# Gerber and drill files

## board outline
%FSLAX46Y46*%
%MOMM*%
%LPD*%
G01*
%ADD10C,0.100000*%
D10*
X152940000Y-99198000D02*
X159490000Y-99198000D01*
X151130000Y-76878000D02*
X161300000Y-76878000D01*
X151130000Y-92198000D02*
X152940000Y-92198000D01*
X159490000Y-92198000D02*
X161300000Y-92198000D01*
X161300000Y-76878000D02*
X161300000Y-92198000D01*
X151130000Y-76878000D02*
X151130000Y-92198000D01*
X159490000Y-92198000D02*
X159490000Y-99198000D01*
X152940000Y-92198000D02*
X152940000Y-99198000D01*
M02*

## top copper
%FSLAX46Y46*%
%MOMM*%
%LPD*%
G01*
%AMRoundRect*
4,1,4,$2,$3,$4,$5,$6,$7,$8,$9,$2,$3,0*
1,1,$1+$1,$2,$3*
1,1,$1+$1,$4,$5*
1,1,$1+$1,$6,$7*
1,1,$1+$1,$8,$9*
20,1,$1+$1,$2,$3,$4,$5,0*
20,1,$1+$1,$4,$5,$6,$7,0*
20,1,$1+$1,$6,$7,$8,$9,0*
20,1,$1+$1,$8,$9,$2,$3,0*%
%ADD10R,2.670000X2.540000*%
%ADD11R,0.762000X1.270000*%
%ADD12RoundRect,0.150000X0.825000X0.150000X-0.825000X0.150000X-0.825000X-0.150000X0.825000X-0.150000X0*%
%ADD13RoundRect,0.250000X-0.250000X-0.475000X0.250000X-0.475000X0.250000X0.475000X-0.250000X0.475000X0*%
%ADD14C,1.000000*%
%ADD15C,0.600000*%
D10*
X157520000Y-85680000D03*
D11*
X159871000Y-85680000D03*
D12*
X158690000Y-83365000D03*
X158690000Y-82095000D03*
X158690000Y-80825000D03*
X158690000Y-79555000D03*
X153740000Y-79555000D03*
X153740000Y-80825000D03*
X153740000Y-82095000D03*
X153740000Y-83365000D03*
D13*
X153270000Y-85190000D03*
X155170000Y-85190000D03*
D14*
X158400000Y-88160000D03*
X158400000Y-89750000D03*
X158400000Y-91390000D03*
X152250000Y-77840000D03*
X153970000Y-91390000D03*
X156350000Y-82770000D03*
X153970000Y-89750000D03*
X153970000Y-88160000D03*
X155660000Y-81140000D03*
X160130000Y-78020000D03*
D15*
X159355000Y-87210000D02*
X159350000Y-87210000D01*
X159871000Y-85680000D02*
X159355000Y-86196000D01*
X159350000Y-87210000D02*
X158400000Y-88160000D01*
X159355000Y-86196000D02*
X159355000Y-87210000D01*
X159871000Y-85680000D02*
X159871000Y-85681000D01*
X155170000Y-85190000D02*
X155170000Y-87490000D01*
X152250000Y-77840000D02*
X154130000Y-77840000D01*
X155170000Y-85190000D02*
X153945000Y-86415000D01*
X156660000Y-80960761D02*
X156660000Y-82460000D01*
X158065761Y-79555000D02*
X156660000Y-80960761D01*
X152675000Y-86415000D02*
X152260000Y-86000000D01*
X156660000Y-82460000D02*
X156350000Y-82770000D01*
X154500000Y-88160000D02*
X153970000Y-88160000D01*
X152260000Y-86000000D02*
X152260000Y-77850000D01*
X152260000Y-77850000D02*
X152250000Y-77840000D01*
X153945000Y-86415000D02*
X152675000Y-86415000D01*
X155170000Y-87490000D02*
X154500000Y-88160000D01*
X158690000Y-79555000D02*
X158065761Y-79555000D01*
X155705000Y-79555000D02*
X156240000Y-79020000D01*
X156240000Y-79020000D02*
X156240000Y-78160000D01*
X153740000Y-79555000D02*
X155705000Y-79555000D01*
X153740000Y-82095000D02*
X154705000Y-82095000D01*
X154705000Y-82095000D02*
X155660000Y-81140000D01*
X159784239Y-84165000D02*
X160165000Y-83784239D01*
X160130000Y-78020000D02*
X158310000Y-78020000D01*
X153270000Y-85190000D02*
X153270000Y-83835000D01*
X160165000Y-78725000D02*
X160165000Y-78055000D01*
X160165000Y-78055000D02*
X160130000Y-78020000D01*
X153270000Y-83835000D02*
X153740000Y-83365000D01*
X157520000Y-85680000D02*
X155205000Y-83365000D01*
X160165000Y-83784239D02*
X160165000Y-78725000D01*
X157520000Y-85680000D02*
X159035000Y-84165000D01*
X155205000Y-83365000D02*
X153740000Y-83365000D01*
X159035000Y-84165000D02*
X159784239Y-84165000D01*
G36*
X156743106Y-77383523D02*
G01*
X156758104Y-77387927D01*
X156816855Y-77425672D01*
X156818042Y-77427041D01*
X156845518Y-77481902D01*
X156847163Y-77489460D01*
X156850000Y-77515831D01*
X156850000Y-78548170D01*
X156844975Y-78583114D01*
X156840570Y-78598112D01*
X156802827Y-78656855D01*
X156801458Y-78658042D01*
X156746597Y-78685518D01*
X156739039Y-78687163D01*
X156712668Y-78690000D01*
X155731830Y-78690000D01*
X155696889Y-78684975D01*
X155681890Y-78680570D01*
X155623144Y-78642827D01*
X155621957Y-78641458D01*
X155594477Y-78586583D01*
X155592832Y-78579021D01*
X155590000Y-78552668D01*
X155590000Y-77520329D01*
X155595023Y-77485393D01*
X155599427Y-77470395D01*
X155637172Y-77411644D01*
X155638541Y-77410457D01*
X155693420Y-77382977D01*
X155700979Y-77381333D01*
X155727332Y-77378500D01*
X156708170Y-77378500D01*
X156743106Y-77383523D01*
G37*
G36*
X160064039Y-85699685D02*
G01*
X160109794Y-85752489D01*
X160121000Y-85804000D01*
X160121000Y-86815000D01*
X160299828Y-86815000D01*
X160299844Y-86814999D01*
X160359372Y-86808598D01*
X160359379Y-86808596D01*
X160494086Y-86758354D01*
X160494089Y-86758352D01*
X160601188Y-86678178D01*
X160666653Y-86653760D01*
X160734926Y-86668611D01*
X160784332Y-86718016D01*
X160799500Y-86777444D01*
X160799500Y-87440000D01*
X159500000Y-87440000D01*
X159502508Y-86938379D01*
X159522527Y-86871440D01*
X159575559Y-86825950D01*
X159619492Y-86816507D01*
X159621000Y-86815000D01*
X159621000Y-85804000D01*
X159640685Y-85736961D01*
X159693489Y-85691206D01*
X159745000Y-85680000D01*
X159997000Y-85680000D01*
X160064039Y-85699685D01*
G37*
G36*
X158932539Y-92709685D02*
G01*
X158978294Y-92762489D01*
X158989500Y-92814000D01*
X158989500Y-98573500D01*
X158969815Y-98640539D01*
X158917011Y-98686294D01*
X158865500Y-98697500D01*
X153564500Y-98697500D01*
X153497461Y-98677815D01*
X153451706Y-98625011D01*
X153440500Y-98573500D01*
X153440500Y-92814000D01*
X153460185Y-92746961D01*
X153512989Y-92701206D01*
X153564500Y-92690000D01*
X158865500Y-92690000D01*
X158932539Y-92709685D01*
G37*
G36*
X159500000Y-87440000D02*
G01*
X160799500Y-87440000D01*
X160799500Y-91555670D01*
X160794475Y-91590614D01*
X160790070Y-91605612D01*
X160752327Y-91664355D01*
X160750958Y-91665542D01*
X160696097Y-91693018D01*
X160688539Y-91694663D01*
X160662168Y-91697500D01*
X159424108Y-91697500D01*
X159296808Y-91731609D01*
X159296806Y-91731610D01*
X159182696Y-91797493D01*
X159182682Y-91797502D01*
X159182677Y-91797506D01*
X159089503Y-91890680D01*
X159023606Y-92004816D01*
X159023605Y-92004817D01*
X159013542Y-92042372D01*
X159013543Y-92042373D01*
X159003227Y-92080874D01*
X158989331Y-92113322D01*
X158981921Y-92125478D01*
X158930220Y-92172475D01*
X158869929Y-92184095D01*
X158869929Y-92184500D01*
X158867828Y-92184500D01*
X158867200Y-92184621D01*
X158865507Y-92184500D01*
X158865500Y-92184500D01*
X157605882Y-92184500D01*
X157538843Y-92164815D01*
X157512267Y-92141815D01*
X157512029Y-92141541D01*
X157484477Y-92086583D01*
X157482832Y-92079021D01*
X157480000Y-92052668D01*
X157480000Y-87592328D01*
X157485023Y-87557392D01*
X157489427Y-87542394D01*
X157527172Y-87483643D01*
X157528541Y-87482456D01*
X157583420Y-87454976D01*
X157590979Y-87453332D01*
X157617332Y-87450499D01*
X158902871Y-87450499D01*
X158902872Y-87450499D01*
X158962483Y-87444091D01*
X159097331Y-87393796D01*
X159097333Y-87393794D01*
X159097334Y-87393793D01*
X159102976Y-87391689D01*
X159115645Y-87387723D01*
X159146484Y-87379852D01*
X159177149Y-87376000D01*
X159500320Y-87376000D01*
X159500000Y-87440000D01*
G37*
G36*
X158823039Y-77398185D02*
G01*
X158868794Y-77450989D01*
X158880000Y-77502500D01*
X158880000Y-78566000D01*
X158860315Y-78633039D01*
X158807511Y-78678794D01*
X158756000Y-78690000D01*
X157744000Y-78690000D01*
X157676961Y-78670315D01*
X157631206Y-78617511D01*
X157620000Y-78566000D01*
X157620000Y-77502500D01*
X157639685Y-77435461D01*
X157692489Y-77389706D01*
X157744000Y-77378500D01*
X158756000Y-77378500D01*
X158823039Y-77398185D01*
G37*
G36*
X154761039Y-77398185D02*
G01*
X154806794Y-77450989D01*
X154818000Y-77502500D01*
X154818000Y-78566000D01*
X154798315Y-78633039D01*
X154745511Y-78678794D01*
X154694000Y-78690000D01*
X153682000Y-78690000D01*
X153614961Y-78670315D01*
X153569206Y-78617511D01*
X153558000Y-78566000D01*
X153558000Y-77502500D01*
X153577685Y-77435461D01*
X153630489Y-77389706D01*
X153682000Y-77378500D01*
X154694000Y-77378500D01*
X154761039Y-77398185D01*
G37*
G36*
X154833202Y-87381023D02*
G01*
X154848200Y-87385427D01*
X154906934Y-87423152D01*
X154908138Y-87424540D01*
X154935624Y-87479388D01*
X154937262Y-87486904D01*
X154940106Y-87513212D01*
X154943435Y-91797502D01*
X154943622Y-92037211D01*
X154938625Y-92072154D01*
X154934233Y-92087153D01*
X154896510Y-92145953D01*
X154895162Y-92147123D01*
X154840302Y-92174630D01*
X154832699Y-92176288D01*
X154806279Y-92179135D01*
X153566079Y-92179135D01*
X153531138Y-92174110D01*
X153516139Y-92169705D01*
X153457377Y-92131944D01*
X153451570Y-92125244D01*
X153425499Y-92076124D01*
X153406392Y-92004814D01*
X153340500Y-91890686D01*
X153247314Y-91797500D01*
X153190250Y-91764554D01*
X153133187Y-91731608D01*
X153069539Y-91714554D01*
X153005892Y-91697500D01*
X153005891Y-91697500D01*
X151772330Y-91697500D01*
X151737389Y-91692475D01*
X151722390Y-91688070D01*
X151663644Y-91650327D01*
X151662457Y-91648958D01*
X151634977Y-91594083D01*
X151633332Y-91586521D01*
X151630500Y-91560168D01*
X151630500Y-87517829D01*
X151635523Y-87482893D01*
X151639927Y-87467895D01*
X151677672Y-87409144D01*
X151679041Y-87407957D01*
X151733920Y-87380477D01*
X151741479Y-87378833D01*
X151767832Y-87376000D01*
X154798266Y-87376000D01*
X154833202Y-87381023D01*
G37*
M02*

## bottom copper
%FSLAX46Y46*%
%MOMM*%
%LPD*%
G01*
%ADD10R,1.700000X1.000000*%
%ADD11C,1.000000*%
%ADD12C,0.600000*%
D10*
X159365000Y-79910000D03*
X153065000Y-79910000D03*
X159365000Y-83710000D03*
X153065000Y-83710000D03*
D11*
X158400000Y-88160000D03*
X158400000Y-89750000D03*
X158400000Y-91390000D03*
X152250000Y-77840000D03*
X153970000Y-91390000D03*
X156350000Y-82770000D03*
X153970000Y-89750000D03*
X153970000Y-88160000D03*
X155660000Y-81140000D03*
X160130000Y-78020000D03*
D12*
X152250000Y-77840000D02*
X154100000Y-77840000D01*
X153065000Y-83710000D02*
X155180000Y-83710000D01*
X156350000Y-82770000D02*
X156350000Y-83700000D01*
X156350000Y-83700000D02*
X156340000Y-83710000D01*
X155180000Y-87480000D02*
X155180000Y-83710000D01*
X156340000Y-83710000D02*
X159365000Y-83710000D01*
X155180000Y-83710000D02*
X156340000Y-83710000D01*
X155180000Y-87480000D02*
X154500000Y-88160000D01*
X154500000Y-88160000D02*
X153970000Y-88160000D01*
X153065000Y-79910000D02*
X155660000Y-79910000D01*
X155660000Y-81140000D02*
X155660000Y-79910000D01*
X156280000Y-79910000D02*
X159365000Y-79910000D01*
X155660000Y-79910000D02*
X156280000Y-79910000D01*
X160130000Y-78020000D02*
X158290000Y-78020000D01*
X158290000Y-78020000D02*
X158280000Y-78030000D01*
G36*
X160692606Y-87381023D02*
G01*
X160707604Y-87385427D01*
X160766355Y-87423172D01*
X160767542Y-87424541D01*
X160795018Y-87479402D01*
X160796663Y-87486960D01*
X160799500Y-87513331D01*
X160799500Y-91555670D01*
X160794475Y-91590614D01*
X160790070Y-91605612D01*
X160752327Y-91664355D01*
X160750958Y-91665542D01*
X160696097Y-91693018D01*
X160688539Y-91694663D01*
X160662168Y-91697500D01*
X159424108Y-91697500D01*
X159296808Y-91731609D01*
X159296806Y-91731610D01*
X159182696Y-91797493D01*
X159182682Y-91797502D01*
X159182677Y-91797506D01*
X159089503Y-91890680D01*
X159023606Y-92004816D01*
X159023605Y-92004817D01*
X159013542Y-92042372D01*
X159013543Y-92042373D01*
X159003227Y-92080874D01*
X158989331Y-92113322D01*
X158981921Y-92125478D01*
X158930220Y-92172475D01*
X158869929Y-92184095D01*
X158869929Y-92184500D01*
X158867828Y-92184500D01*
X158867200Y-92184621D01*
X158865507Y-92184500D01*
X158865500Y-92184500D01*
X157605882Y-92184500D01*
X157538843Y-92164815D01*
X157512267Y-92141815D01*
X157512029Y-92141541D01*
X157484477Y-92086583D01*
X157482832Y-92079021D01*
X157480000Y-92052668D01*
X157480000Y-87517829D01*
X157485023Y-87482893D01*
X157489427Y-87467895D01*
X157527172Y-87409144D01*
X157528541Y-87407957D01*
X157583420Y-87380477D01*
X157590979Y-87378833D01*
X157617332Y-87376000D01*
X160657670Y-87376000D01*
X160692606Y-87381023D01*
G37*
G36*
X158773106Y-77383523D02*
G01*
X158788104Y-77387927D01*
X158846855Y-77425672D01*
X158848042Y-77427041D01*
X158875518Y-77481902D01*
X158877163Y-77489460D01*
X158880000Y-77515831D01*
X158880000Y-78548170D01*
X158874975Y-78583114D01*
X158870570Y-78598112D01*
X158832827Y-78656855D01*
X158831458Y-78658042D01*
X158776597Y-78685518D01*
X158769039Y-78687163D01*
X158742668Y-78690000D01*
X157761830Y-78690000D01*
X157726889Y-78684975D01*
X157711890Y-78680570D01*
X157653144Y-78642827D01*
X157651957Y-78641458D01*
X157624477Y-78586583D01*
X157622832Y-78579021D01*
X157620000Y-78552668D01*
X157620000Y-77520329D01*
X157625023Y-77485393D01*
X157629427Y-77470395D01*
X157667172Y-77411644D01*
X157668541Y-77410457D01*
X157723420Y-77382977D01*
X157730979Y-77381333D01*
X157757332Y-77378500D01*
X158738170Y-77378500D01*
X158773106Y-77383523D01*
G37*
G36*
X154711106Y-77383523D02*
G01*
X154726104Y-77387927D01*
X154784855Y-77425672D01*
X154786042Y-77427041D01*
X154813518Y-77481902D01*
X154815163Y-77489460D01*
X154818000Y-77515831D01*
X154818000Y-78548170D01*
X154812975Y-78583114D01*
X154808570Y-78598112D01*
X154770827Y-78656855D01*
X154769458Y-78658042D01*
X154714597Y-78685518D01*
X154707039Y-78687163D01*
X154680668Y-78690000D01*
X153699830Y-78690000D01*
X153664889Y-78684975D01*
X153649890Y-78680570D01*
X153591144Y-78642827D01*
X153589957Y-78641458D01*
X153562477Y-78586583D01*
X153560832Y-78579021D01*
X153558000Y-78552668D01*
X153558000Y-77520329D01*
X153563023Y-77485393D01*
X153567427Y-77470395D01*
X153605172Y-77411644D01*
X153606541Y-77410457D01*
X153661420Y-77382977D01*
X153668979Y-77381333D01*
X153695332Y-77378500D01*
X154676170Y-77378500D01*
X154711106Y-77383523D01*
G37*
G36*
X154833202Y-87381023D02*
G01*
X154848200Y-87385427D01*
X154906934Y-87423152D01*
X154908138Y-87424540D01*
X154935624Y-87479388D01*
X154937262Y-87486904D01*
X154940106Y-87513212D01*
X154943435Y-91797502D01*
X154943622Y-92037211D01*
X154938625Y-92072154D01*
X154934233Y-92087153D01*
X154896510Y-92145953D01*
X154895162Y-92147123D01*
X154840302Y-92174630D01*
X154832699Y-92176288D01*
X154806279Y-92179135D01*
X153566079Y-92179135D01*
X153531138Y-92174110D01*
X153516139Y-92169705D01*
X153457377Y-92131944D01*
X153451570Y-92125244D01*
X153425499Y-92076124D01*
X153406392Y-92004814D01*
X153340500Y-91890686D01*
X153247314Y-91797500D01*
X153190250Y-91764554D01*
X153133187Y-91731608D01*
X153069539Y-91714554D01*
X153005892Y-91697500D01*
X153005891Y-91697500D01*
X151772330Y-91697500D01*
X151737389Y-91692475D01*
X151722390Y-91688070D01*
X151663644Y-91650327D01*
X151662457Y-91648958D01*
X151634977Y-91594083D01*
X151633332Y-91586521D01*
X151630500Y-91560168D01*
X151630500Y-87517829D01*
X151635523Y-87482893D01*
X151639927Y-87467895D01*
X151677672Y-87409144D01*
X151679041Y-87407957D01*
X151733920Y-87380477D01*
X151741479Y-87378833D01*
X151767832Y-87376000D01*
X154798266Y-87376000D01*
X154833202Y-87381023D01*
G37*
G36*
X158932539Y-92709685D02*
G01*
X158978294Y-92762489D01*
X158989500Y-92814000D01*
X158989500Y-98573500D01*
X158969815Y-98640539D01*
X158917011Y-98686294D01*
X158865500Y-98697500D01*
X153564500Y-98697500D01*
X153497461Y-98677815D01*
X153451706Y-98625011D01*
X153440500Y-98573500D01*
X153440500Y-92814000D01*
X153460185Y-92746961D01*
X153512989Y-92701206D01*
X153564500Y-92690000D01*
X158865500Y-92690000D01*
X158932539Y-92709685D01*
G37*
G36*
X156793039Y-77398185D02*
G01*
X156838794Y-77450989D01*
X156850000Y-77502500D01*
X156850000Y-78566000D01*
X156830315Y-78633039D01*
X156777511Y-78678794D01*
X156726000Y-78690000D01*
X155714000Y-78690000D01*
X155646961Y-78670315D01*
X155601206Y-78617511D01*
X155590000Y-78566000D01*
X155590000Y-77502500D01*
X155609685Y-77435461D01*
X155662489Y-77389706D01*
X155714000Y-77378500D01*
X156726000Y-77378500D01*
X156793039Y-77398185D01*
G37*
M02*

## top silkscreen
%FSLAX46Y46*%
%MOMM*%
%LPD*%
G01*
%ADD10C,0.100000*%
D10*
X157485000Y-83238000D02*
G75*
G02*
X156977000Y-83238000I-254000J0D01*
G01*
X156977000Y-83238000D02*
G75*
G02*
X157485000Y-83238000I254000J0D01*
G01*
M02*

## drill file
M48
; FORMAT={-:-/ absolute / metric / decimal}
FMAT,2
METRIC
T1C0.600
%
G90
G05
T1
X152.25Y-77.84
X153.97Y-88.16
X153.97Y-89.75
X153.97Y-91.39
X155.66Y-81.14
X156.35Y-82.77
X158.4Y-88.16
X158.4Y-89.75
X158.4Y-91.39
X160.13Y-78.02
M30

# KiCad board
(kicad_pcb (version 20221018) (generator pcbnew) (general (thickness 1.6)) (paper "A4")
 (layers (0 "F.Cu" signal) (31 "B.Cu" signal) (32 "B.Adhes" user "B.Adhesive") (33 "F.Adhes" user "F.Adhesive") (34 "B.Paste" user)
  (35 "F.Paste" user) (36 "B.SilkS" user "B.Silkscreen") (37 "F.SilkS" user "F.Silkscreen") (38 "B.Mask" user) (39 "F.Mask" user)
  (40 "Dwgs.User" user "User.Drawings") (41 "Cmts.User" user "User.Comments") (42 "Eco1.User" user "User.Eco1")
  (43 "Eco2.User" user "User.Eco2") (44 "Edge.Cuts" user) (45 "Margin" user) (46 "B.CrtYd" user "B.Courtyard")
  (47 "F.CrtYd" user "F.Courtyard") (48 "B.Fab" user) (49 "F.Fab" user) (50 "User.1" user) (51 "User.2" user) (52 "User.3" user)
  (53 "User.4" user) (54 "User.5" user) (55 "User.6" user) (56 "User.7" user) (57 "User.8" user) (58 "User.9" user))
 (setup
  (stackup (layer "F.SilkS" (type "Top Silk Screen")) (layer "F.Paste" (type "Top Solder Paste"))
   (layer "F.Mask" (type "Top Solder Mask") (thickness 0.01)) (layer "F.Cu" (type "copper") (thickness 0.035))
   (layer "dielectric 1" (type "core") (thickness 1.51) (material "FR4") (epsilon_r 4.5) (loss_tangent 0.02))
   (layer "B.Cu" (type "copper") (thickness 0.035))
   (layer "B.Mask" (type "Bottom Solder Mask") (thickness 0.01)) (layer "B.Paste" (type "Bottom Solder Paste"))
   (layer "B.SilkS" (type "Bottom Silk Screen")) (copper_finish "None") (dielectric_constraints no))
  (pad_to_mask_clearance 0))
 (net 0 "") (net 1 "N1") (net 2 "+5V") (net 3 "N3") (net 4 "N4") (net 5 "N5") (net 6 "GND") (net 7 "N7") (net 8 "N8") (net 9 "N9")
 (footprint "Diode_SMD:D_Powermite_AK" (layer "F.Cu") (at 158.2185 85.68)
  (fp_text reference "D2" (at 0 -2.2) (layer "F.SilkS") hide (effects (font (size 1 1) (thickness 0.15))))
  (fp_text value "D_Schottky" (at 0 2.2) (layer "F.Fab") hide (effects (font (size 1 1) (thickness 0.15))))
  (pad "1" smd rect (at -0.6985 0) (size 2.67 2.54) (layers "F.Cu" "F.Paste" "F.Mask") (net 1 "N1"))
  (pad "2" smd rect (at 1.6525 0) (size 0.762 1.27) (layers "F.Cu" "F.Paste" "F.Mask") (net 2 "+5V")))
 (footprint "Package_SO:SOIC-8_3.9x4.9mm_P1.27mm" (layer "F.Cu") (at 156.215 81.46 180)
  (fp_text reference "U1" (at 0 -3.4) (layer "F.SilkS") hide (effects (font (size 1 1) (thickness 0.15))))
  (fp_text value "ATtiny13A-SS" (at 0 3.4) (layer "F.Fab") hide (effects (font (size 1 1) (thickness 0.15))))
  (fp_circle (center -1.016 -1.778) (end -0.762 -1.778) (stroke (width 0.1) (type default)) (fill none) (layer "F.SilkS"))
  (pad "1" smd roundrect (at -2.475 -1.905 180) (size 1.95 0.6) (layers "F.Cu" "F.Paste" "F.Mask") (roundrect_rratio 0.25) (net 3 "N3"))
  (pad "2" smd roundrect (at -2.475 -0.635 180) (size 1.95 0.6) (layers "F.Cu" "F.Paste" "F.Mask") (roundrect_rratio 0.25) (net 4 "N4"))
  (pad "3" smd roundrect (at -2.475 0.635 180) (size 1.95 0.6) (layers "F.Cu" "F.Paste" "F.Mask") (roundrect_rratio 0.25) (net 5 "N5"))
  (pad "4" smd roundrect (at -2.475 1.905 180) (size 1.95 0.6) (layers "F.Cu" "F.Paste" "F.Mask") (roundrect_rratio 0.25) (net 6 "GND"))
  (pad "5" smd roundrect (at 2.475 1.905 180) (size 1.95 0.6) (layers "F.Cu" "F.Paste" "F.Mask") (roundrect_rratio 0.25) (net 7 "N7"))
  (pad "6" smd roundrect (at 2.475 0.635 180) (size 1.95 0.6) (layers "F.Cu" "F.Paste" "F.Mask") (roundrect_rratio 0.25) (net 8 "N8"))
  (pad "7" smd roundrect (at 2.475 -0.635 180) (size 1.95 0.6) (layers "F.Cu" "F.Paste" "F.Mask") (roundrect_rratio 0.25) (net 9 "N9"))
  (pad "8" smd roundrect (at 2.475 -1.905 180) (size 1.95 0.6) (layers "F.Cu" "F.Paste" "F.Mask") (roundrect_rratio 0.25) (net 1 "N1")))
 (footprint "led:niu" (layer "F.Cu") (at 156.038877 95.899084)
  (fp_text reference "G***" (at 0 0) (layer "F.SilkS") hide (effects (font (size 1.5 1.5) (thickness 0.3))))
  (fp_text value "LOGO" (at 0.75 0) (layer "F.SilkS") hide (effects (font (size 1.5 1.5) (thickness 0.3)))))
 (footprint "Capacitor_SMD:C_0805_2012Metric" (layer "F.Cu") (at 154.22 85.19)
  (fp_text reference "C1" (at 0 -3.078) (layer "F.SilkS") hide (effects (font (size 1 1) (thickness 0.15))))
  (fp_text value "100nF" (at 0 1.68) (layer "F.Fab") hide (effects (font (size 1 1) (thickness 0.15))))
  (pad "1" smd roundrect (at -0.95 0) (size 1 1.45) (layers "F.Cu" "F.Paste" "F.Mask") (roundrect_rratio 0.25) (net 1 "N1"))
  (pad "2" smd roundrect (at 0.95 0) (size 1 1.45) (layers "F.Cu" "F.Paste" "F.Mask") (roundrect_rratio 0.25) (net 6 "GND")))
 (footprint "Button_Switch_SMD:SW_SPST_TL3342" (layer "B.Cu") (at 156.215 81.81 180)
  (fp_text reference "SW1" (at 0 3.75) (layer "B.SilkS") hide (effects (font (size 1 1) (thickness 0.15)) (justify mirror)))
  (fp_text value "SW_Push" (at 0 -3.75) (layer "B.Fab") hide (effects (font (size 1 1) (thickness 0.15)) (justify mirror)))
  (pad "1" smd rect (at -3.15 1.9 180) (size 1.7 1) (layers "B.Cu" "B.Paste" "B.Mask") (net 9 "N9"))
  (pad "1" smd rect (at 3.15 1.9 180) (size 1.7 1) (layers "B.Cu" "B.Paste" "B.Mask") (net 9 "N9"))
  (pad "2" smd rect (at -3.15 -1.9 180) (size 1.7 1) (layers "B.Cu" "B.Paste" "B.Mask") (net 6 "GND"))
  (pad "2" smd rect (at 3.15 -1.9 180) (size 1.7 1) (layers "B.Cu" "B.Paste" "B.Mask") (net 6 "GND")))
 (gr_line (start 152.94 99.198) (end 159.49 99.198) (stroke (width 0.1) (type default)) (layer "Edge.Cuts"))
 (gr_line (start 151.13 76.878) (end 161.3 76.878) (stroke (width 0.1) (type default)) (layer "Edge.Cuts"))
 (gr_line (start 151.13 92.198) (end 152.94 92.198) (stroke (width 0.1) (type default)) (layer "Edge.Cuts"))
 (gr_line (start 159.49 92.198) (end 161.3 92.198) (stroke (width 0.1) (type default)) (layer "Edge.Cuts"))
 (gr_line (start 161.3 76.878) (end 161.3 92.198) (stroke (width 0.1) (type default)) (layer "Edge.Cuts"))
 (gr_line (start 151.13 76.878) (end 151.13 92.198) (stroke (width 0.1) (type default)) (layer "Edge.Cuts"))
 (gr_line (start 159.49 92.198) (end 159.49 99.198) (stroke (width 0.1) (type default)) (layer "Edge.Cuts"))
 (gr_line (start 152.94 92.198) (end 152.94 99.198) (stroke (width 0.1) (type default)) (layer "Edge.Cuts"))
 (segment (start 159.355 87.21) (end 159.35 87.21) (width 0.6) (layer "F.Cu") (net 2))
 (segment (start 159.871 85.68) (end 159.355 86.196) (width 0.6) (layer "F.Cu") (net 2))
 (segment (start 159.35 87.21) (end 158.4 88.16) (width 0.6) (layer "F.Cu") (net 2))
 (segment (start 159.355 86.196) (end 159.355 87.21) (width 0.6) (layer "F.Cu") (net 2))
 (segment (start 159.871 85.68) (end 159.871 85.681) (width 0.6) (layer "F.Cu") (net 2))
 (via (at 158.4 88.16) (size 1) (drill 0.6) (layers "F.Cu" "B.Cu") (free) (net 2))
 (via (at 158.4 89.75) (size 1) (drill 0.6) (layers "F.Cu" "B.Cu") (free) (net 2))
 (via (at 158.4 91.39) (size 1) (drill 0.6) (layers "F.Cu" "B.Cu") (free) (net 2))
 (segment (start 155.17 85.19) (end 155.17 87.49) (width 0.6) (layer "F.Cu") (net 6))
 (segment (start 152.25 77.84) (end 154.13 77.84) (width 0.6) (layer "F.Cu") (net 6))
 (segment (start 155.17 85.19) (end 153.945 86.415) (width 0.6) (layer "F.Cu") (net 6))
 (segment (start 156.66 80.960761) (end 156.66 82.46) (width 0.6) (layer "F.Cu") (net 6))
 (segment (start 158.065761 79.555) (end 156.66 80.960761) (width 0.6) (layer "F.Cu") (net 6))
 (segment (start 152.675 86.415) (end 152.26 86) (width 0.6) (layer "F.Cu") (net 6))
 (segment (start 156.66 82.46) (end 156.35 82.77) (width 0.6) (layer "F.Cu") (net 6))
 (segment (start 154.5 88.16) (end 153.97 88.16) (width 0.6) (layer "F.Cu") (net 6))
 (segment (start 152.26 86) (end 152.26 77.85) (width 0.6) (layer "F.Cu") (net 6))
 (segment (start 152.26 77.85) (end 152.25 77.84) (width 0.6) (layer "F.Cu") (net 6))
 (segment (start 153.945 86.415) (end 152.675 86.415) (width 0.6) (layer "F.Cu") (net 6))
 (segment (start 155.17 87.49) (end 154.5 88.16) (width 0.6) (layer "F.Cu") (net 6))
 (segment (start 158.69 79.555) (end 158.065761 79.555) (width 0.6) (layer "F.Cu") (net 6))
 (via (at 152.25 77.84) (size 1) (drill 0.6) (layers "F.Cu" "B.Cu") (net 6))
 (via (at 153.97 91.39) (size 1) (drill 0.6) (layers "F.Cu" "B.Cu") (free) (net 6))
 (via (at 156.35 82.77) (size 1) (drill 0.6) (layers "F.Cu" "B.Cu") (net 6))
 (via (at 153.97 89.75) (size 1) (drill 0.6) (layers "F.Cu" "B.Cu") (free) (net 6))
 (via (at 153.97 88.16) (size 1) (drill 0.6) (layers "F.Cu" "B.Cu") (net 6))
 (segment (start 152.25 77.84) (end 154.1 77.84) (width 0.6) (layer "B.Cu") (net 6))
 (segment (start 153.065 83.71) (end 155.18 83.71) (width 0.6) (layer "B.Cu") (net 6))
 (segment (start 156.35 82.77) (end 156.35 83.7) (width 0.6) (layer "B.Cu") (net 6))
 (segment (start 156.35 83.7) (end 156.34 83.71) (width 0.6) (layer "B.Cu") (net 6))
 (segment (start 155.18 87.48) (end 155.18 83.71) (width 0.6) (layer "B.Cu") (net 6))
 (segment (start 156.34 83.71) (end 159.365 83.71) (width 0.6) (layer "B.Cu") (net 6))
 (segment (start 155.18 83.71) (end 156.34 83.71) (width 0.6) (layer "B.Cu") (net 6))
 (segment (start 155.18 87.48) (end 154.5 88.16) (width 0.6) (layer "B.Cu") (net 6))
 (segment (start 154.5 88.16) (end 153.97 88.16) (width 0.6) (layer "B.Cu") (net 6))
 (segment (start 155.705 79.555) (end 156.24 79.02) (width 0.6) (layer "F.Cu") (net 7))
 (segment (start 156.24 79.02) (end 156.24 78.16) (width 0.6) (layer "F.Cu") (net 7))
 (segment (start 153.74 79.555) (end 155.705 79.555) (width 0.6) (layer "F.Cu") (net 7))
 (segment (start 153.74 82.095) (end 154.705 82.095) (width 0.6) (layer "F.Cu") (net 9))
 (segment (start 154.705 82.095) (end 155.66 81.14) (width 0.6) (layer "F.Cu") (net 9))
 (via (at 155.66 81.14) (size 1) (drill 0.6) (layers "F.Cu" "B.Cu") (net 9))
 (segment (start 153.065 79.91) (end 155.66 79.91) (width 0.6) (layer "B.Cu") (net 9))
 (segment (start 155.66 81.14) (end 155.66 79.91) (width 0.6) (layer "B.Cu") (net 9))
 (segment (start 156.28 79.91) (end 159.365 79.91) (width 0.6) (layer "B.Cu") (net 9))
 (segment (start 155.66 79.91) (end 156.28 79.91) (width 0.6) (layer "B.Cu") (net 9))
 (segment (start 159.784239 84.165) (end 160.165 83.784239) (width 0.6) (layer "F.Cu") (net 1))
 (segment (start 160.13 78.02) (end 158.31 78.02) (width 0.6) (layer "F.Cu") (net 1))
 (segment (start 153.27 85.19) (end 153.27 83.835) (width 0.6) (layer "F.Cu") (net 1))
 (segment (start 160.165 78.725) (end 160.165 78.055) (width 0.6) (layer "F.Cu") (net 1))
 (segment (start 160.165 78.055) (end 160.13 78.02) (width 0.6) (layer "F.Cu") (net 1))
 (segment (start 153.27 83.835) (end 153.74 83.365) (width 0.6) (layer "F.Cu") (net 1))
 (segment (start 157.52 85.68) (end 155.205 83.365) (width 0.6) (layer "F.Cu") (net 1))
 (segment (start 160.165 83.784239) (end 160.165 78.725) (width 0.6) (layer "F.Cu") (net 1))
 (segment (start 157.52 85.68) (end 159.035 84.165) (width 0.6) (layer "F.Cu") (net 1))
 (segment (start 155.205 83.365) (end 153.74 83.365) (width 0.6) (layer "F.Cu") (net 1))
 (segment (start 159.035 84.165) (end 159.784239 84.165) (width 0.6) (layer "F.Cu") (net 1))
 (via (at 160.13 78.02) (size 1) (drill 0.6) (layers "F.Cu" "B.Cu") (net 1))
 (segment (start 160.13 78.02) (end 158.29 78.02) (width 0.6) (layer "B.Cu") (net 1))
 (segment (start 158.29 78.02) (end 158.28 78.03) (width 0.6) (layer "B.Cu") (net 1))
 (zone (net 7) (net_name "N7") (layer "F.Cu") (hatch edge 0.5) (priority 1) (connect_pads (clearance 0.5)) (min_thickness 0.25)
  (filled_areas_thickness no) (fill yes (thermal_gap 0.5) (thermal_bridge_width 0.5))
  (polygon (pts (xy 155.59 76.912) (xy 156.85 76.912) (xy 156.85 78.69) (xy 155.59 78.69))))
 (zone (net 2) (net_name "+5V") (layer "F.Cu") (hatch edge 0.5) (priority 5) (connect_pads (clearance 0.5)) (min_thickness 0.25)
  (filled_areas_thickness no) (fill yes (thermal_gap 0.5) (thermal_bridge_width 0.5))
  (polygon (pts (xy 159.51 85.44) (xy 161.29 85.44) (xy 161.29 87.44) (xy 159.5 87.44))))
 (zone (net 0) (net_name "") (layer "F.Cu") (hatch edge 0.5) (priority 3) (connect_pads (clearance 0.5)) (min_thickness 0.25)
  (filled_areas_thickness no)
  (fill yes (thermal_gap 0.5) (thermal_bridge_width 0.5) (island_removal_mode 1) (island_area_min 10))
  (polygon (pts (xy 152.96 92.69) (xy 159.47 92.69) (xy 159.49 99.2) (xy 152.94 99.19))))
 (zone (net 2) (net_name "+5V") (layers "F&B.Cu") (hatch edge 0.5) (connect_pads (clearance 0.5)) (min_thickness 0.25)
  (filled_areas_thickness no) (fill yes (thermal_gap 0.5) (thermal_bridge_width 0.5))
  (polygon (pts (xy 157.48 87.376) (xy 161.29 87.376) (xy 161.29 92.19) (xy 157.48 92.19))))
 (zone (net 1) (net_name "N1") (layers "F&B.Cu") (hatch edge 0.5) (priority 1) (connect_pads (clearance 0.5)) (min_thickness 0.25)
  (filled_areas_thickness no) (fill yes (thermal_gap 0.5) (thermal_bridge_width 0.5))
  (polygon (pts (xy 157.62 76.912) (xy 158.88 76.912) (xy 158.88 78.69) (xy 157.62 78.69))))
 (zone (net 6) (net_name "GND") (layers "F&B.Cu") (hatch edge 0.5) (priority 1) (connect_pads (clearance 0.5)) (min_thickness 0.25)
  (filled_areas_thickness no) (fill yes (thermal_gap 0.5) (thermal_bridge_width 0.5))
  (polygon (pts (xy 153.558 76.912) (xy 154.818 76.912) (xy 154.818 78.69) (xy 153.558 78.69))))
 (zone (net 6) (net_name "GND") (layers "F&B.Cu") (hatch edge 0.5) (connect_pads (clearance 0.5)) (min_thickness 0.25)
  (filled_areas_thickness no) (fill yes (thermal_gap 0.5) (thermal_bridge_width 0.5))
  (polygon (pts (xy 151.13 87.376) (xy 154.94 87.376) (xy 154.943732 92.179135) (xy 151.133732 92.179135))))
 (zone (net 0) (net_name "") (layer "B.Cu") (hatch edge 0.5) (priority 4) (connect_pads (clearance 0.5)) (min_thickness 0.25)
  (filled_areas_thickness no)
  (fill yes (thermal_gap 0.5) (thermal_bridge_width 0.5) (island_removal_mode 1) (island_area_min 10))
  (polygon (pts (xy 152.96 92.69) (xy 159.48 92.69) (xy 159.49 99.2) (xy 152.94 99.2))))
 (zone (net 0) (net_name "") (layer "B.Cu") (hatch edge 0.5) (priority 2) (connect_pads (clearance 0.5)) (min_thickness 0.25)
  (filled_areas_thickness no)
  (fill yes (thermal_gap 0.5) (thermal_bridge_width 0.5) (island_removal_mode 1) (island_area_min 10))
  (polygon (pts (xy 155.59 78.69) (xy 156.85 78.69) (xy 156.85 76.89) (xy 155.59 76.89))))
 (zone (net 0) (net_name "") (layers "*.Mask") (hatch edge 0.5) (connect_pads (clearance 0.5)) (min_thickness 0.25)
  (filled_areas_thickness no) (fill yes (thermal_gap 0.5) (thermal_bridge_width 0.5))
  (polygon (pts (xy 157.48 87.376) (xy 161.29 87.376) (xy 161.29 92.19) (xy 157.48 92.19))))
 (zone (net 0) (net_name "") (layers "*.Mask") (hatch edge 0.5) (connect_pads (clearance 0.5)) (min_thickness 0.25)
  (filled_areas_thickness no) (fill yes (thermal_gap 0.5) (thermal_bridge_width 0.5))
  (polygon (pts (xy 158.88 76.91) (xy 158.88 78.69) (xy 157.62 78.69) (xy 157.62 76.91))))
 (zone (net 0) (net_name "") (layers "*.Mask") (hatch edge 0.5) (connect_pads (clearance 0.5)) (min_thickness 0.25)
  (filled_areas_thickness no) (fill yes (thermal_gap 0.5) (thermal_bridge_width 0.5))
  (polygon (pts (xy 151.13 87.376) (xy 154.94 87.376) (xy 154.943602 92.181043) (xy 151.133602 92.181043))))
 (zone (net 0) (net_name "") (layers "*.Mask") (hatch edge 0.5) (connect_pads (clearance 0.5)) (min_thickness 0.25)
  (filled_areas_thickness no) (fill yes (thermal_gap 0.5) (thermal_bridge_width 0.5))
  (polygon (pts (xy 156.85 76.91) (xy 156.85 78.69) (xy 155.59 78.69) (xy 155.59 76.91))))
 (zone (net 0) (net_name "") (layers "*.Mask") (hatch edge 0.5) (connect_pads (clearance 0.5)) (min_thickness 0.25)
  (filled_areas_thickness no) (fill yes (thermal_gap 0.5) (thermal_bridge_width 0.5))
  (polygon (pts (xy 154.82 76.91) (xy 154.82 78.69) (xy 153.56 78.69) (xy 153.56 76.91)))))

